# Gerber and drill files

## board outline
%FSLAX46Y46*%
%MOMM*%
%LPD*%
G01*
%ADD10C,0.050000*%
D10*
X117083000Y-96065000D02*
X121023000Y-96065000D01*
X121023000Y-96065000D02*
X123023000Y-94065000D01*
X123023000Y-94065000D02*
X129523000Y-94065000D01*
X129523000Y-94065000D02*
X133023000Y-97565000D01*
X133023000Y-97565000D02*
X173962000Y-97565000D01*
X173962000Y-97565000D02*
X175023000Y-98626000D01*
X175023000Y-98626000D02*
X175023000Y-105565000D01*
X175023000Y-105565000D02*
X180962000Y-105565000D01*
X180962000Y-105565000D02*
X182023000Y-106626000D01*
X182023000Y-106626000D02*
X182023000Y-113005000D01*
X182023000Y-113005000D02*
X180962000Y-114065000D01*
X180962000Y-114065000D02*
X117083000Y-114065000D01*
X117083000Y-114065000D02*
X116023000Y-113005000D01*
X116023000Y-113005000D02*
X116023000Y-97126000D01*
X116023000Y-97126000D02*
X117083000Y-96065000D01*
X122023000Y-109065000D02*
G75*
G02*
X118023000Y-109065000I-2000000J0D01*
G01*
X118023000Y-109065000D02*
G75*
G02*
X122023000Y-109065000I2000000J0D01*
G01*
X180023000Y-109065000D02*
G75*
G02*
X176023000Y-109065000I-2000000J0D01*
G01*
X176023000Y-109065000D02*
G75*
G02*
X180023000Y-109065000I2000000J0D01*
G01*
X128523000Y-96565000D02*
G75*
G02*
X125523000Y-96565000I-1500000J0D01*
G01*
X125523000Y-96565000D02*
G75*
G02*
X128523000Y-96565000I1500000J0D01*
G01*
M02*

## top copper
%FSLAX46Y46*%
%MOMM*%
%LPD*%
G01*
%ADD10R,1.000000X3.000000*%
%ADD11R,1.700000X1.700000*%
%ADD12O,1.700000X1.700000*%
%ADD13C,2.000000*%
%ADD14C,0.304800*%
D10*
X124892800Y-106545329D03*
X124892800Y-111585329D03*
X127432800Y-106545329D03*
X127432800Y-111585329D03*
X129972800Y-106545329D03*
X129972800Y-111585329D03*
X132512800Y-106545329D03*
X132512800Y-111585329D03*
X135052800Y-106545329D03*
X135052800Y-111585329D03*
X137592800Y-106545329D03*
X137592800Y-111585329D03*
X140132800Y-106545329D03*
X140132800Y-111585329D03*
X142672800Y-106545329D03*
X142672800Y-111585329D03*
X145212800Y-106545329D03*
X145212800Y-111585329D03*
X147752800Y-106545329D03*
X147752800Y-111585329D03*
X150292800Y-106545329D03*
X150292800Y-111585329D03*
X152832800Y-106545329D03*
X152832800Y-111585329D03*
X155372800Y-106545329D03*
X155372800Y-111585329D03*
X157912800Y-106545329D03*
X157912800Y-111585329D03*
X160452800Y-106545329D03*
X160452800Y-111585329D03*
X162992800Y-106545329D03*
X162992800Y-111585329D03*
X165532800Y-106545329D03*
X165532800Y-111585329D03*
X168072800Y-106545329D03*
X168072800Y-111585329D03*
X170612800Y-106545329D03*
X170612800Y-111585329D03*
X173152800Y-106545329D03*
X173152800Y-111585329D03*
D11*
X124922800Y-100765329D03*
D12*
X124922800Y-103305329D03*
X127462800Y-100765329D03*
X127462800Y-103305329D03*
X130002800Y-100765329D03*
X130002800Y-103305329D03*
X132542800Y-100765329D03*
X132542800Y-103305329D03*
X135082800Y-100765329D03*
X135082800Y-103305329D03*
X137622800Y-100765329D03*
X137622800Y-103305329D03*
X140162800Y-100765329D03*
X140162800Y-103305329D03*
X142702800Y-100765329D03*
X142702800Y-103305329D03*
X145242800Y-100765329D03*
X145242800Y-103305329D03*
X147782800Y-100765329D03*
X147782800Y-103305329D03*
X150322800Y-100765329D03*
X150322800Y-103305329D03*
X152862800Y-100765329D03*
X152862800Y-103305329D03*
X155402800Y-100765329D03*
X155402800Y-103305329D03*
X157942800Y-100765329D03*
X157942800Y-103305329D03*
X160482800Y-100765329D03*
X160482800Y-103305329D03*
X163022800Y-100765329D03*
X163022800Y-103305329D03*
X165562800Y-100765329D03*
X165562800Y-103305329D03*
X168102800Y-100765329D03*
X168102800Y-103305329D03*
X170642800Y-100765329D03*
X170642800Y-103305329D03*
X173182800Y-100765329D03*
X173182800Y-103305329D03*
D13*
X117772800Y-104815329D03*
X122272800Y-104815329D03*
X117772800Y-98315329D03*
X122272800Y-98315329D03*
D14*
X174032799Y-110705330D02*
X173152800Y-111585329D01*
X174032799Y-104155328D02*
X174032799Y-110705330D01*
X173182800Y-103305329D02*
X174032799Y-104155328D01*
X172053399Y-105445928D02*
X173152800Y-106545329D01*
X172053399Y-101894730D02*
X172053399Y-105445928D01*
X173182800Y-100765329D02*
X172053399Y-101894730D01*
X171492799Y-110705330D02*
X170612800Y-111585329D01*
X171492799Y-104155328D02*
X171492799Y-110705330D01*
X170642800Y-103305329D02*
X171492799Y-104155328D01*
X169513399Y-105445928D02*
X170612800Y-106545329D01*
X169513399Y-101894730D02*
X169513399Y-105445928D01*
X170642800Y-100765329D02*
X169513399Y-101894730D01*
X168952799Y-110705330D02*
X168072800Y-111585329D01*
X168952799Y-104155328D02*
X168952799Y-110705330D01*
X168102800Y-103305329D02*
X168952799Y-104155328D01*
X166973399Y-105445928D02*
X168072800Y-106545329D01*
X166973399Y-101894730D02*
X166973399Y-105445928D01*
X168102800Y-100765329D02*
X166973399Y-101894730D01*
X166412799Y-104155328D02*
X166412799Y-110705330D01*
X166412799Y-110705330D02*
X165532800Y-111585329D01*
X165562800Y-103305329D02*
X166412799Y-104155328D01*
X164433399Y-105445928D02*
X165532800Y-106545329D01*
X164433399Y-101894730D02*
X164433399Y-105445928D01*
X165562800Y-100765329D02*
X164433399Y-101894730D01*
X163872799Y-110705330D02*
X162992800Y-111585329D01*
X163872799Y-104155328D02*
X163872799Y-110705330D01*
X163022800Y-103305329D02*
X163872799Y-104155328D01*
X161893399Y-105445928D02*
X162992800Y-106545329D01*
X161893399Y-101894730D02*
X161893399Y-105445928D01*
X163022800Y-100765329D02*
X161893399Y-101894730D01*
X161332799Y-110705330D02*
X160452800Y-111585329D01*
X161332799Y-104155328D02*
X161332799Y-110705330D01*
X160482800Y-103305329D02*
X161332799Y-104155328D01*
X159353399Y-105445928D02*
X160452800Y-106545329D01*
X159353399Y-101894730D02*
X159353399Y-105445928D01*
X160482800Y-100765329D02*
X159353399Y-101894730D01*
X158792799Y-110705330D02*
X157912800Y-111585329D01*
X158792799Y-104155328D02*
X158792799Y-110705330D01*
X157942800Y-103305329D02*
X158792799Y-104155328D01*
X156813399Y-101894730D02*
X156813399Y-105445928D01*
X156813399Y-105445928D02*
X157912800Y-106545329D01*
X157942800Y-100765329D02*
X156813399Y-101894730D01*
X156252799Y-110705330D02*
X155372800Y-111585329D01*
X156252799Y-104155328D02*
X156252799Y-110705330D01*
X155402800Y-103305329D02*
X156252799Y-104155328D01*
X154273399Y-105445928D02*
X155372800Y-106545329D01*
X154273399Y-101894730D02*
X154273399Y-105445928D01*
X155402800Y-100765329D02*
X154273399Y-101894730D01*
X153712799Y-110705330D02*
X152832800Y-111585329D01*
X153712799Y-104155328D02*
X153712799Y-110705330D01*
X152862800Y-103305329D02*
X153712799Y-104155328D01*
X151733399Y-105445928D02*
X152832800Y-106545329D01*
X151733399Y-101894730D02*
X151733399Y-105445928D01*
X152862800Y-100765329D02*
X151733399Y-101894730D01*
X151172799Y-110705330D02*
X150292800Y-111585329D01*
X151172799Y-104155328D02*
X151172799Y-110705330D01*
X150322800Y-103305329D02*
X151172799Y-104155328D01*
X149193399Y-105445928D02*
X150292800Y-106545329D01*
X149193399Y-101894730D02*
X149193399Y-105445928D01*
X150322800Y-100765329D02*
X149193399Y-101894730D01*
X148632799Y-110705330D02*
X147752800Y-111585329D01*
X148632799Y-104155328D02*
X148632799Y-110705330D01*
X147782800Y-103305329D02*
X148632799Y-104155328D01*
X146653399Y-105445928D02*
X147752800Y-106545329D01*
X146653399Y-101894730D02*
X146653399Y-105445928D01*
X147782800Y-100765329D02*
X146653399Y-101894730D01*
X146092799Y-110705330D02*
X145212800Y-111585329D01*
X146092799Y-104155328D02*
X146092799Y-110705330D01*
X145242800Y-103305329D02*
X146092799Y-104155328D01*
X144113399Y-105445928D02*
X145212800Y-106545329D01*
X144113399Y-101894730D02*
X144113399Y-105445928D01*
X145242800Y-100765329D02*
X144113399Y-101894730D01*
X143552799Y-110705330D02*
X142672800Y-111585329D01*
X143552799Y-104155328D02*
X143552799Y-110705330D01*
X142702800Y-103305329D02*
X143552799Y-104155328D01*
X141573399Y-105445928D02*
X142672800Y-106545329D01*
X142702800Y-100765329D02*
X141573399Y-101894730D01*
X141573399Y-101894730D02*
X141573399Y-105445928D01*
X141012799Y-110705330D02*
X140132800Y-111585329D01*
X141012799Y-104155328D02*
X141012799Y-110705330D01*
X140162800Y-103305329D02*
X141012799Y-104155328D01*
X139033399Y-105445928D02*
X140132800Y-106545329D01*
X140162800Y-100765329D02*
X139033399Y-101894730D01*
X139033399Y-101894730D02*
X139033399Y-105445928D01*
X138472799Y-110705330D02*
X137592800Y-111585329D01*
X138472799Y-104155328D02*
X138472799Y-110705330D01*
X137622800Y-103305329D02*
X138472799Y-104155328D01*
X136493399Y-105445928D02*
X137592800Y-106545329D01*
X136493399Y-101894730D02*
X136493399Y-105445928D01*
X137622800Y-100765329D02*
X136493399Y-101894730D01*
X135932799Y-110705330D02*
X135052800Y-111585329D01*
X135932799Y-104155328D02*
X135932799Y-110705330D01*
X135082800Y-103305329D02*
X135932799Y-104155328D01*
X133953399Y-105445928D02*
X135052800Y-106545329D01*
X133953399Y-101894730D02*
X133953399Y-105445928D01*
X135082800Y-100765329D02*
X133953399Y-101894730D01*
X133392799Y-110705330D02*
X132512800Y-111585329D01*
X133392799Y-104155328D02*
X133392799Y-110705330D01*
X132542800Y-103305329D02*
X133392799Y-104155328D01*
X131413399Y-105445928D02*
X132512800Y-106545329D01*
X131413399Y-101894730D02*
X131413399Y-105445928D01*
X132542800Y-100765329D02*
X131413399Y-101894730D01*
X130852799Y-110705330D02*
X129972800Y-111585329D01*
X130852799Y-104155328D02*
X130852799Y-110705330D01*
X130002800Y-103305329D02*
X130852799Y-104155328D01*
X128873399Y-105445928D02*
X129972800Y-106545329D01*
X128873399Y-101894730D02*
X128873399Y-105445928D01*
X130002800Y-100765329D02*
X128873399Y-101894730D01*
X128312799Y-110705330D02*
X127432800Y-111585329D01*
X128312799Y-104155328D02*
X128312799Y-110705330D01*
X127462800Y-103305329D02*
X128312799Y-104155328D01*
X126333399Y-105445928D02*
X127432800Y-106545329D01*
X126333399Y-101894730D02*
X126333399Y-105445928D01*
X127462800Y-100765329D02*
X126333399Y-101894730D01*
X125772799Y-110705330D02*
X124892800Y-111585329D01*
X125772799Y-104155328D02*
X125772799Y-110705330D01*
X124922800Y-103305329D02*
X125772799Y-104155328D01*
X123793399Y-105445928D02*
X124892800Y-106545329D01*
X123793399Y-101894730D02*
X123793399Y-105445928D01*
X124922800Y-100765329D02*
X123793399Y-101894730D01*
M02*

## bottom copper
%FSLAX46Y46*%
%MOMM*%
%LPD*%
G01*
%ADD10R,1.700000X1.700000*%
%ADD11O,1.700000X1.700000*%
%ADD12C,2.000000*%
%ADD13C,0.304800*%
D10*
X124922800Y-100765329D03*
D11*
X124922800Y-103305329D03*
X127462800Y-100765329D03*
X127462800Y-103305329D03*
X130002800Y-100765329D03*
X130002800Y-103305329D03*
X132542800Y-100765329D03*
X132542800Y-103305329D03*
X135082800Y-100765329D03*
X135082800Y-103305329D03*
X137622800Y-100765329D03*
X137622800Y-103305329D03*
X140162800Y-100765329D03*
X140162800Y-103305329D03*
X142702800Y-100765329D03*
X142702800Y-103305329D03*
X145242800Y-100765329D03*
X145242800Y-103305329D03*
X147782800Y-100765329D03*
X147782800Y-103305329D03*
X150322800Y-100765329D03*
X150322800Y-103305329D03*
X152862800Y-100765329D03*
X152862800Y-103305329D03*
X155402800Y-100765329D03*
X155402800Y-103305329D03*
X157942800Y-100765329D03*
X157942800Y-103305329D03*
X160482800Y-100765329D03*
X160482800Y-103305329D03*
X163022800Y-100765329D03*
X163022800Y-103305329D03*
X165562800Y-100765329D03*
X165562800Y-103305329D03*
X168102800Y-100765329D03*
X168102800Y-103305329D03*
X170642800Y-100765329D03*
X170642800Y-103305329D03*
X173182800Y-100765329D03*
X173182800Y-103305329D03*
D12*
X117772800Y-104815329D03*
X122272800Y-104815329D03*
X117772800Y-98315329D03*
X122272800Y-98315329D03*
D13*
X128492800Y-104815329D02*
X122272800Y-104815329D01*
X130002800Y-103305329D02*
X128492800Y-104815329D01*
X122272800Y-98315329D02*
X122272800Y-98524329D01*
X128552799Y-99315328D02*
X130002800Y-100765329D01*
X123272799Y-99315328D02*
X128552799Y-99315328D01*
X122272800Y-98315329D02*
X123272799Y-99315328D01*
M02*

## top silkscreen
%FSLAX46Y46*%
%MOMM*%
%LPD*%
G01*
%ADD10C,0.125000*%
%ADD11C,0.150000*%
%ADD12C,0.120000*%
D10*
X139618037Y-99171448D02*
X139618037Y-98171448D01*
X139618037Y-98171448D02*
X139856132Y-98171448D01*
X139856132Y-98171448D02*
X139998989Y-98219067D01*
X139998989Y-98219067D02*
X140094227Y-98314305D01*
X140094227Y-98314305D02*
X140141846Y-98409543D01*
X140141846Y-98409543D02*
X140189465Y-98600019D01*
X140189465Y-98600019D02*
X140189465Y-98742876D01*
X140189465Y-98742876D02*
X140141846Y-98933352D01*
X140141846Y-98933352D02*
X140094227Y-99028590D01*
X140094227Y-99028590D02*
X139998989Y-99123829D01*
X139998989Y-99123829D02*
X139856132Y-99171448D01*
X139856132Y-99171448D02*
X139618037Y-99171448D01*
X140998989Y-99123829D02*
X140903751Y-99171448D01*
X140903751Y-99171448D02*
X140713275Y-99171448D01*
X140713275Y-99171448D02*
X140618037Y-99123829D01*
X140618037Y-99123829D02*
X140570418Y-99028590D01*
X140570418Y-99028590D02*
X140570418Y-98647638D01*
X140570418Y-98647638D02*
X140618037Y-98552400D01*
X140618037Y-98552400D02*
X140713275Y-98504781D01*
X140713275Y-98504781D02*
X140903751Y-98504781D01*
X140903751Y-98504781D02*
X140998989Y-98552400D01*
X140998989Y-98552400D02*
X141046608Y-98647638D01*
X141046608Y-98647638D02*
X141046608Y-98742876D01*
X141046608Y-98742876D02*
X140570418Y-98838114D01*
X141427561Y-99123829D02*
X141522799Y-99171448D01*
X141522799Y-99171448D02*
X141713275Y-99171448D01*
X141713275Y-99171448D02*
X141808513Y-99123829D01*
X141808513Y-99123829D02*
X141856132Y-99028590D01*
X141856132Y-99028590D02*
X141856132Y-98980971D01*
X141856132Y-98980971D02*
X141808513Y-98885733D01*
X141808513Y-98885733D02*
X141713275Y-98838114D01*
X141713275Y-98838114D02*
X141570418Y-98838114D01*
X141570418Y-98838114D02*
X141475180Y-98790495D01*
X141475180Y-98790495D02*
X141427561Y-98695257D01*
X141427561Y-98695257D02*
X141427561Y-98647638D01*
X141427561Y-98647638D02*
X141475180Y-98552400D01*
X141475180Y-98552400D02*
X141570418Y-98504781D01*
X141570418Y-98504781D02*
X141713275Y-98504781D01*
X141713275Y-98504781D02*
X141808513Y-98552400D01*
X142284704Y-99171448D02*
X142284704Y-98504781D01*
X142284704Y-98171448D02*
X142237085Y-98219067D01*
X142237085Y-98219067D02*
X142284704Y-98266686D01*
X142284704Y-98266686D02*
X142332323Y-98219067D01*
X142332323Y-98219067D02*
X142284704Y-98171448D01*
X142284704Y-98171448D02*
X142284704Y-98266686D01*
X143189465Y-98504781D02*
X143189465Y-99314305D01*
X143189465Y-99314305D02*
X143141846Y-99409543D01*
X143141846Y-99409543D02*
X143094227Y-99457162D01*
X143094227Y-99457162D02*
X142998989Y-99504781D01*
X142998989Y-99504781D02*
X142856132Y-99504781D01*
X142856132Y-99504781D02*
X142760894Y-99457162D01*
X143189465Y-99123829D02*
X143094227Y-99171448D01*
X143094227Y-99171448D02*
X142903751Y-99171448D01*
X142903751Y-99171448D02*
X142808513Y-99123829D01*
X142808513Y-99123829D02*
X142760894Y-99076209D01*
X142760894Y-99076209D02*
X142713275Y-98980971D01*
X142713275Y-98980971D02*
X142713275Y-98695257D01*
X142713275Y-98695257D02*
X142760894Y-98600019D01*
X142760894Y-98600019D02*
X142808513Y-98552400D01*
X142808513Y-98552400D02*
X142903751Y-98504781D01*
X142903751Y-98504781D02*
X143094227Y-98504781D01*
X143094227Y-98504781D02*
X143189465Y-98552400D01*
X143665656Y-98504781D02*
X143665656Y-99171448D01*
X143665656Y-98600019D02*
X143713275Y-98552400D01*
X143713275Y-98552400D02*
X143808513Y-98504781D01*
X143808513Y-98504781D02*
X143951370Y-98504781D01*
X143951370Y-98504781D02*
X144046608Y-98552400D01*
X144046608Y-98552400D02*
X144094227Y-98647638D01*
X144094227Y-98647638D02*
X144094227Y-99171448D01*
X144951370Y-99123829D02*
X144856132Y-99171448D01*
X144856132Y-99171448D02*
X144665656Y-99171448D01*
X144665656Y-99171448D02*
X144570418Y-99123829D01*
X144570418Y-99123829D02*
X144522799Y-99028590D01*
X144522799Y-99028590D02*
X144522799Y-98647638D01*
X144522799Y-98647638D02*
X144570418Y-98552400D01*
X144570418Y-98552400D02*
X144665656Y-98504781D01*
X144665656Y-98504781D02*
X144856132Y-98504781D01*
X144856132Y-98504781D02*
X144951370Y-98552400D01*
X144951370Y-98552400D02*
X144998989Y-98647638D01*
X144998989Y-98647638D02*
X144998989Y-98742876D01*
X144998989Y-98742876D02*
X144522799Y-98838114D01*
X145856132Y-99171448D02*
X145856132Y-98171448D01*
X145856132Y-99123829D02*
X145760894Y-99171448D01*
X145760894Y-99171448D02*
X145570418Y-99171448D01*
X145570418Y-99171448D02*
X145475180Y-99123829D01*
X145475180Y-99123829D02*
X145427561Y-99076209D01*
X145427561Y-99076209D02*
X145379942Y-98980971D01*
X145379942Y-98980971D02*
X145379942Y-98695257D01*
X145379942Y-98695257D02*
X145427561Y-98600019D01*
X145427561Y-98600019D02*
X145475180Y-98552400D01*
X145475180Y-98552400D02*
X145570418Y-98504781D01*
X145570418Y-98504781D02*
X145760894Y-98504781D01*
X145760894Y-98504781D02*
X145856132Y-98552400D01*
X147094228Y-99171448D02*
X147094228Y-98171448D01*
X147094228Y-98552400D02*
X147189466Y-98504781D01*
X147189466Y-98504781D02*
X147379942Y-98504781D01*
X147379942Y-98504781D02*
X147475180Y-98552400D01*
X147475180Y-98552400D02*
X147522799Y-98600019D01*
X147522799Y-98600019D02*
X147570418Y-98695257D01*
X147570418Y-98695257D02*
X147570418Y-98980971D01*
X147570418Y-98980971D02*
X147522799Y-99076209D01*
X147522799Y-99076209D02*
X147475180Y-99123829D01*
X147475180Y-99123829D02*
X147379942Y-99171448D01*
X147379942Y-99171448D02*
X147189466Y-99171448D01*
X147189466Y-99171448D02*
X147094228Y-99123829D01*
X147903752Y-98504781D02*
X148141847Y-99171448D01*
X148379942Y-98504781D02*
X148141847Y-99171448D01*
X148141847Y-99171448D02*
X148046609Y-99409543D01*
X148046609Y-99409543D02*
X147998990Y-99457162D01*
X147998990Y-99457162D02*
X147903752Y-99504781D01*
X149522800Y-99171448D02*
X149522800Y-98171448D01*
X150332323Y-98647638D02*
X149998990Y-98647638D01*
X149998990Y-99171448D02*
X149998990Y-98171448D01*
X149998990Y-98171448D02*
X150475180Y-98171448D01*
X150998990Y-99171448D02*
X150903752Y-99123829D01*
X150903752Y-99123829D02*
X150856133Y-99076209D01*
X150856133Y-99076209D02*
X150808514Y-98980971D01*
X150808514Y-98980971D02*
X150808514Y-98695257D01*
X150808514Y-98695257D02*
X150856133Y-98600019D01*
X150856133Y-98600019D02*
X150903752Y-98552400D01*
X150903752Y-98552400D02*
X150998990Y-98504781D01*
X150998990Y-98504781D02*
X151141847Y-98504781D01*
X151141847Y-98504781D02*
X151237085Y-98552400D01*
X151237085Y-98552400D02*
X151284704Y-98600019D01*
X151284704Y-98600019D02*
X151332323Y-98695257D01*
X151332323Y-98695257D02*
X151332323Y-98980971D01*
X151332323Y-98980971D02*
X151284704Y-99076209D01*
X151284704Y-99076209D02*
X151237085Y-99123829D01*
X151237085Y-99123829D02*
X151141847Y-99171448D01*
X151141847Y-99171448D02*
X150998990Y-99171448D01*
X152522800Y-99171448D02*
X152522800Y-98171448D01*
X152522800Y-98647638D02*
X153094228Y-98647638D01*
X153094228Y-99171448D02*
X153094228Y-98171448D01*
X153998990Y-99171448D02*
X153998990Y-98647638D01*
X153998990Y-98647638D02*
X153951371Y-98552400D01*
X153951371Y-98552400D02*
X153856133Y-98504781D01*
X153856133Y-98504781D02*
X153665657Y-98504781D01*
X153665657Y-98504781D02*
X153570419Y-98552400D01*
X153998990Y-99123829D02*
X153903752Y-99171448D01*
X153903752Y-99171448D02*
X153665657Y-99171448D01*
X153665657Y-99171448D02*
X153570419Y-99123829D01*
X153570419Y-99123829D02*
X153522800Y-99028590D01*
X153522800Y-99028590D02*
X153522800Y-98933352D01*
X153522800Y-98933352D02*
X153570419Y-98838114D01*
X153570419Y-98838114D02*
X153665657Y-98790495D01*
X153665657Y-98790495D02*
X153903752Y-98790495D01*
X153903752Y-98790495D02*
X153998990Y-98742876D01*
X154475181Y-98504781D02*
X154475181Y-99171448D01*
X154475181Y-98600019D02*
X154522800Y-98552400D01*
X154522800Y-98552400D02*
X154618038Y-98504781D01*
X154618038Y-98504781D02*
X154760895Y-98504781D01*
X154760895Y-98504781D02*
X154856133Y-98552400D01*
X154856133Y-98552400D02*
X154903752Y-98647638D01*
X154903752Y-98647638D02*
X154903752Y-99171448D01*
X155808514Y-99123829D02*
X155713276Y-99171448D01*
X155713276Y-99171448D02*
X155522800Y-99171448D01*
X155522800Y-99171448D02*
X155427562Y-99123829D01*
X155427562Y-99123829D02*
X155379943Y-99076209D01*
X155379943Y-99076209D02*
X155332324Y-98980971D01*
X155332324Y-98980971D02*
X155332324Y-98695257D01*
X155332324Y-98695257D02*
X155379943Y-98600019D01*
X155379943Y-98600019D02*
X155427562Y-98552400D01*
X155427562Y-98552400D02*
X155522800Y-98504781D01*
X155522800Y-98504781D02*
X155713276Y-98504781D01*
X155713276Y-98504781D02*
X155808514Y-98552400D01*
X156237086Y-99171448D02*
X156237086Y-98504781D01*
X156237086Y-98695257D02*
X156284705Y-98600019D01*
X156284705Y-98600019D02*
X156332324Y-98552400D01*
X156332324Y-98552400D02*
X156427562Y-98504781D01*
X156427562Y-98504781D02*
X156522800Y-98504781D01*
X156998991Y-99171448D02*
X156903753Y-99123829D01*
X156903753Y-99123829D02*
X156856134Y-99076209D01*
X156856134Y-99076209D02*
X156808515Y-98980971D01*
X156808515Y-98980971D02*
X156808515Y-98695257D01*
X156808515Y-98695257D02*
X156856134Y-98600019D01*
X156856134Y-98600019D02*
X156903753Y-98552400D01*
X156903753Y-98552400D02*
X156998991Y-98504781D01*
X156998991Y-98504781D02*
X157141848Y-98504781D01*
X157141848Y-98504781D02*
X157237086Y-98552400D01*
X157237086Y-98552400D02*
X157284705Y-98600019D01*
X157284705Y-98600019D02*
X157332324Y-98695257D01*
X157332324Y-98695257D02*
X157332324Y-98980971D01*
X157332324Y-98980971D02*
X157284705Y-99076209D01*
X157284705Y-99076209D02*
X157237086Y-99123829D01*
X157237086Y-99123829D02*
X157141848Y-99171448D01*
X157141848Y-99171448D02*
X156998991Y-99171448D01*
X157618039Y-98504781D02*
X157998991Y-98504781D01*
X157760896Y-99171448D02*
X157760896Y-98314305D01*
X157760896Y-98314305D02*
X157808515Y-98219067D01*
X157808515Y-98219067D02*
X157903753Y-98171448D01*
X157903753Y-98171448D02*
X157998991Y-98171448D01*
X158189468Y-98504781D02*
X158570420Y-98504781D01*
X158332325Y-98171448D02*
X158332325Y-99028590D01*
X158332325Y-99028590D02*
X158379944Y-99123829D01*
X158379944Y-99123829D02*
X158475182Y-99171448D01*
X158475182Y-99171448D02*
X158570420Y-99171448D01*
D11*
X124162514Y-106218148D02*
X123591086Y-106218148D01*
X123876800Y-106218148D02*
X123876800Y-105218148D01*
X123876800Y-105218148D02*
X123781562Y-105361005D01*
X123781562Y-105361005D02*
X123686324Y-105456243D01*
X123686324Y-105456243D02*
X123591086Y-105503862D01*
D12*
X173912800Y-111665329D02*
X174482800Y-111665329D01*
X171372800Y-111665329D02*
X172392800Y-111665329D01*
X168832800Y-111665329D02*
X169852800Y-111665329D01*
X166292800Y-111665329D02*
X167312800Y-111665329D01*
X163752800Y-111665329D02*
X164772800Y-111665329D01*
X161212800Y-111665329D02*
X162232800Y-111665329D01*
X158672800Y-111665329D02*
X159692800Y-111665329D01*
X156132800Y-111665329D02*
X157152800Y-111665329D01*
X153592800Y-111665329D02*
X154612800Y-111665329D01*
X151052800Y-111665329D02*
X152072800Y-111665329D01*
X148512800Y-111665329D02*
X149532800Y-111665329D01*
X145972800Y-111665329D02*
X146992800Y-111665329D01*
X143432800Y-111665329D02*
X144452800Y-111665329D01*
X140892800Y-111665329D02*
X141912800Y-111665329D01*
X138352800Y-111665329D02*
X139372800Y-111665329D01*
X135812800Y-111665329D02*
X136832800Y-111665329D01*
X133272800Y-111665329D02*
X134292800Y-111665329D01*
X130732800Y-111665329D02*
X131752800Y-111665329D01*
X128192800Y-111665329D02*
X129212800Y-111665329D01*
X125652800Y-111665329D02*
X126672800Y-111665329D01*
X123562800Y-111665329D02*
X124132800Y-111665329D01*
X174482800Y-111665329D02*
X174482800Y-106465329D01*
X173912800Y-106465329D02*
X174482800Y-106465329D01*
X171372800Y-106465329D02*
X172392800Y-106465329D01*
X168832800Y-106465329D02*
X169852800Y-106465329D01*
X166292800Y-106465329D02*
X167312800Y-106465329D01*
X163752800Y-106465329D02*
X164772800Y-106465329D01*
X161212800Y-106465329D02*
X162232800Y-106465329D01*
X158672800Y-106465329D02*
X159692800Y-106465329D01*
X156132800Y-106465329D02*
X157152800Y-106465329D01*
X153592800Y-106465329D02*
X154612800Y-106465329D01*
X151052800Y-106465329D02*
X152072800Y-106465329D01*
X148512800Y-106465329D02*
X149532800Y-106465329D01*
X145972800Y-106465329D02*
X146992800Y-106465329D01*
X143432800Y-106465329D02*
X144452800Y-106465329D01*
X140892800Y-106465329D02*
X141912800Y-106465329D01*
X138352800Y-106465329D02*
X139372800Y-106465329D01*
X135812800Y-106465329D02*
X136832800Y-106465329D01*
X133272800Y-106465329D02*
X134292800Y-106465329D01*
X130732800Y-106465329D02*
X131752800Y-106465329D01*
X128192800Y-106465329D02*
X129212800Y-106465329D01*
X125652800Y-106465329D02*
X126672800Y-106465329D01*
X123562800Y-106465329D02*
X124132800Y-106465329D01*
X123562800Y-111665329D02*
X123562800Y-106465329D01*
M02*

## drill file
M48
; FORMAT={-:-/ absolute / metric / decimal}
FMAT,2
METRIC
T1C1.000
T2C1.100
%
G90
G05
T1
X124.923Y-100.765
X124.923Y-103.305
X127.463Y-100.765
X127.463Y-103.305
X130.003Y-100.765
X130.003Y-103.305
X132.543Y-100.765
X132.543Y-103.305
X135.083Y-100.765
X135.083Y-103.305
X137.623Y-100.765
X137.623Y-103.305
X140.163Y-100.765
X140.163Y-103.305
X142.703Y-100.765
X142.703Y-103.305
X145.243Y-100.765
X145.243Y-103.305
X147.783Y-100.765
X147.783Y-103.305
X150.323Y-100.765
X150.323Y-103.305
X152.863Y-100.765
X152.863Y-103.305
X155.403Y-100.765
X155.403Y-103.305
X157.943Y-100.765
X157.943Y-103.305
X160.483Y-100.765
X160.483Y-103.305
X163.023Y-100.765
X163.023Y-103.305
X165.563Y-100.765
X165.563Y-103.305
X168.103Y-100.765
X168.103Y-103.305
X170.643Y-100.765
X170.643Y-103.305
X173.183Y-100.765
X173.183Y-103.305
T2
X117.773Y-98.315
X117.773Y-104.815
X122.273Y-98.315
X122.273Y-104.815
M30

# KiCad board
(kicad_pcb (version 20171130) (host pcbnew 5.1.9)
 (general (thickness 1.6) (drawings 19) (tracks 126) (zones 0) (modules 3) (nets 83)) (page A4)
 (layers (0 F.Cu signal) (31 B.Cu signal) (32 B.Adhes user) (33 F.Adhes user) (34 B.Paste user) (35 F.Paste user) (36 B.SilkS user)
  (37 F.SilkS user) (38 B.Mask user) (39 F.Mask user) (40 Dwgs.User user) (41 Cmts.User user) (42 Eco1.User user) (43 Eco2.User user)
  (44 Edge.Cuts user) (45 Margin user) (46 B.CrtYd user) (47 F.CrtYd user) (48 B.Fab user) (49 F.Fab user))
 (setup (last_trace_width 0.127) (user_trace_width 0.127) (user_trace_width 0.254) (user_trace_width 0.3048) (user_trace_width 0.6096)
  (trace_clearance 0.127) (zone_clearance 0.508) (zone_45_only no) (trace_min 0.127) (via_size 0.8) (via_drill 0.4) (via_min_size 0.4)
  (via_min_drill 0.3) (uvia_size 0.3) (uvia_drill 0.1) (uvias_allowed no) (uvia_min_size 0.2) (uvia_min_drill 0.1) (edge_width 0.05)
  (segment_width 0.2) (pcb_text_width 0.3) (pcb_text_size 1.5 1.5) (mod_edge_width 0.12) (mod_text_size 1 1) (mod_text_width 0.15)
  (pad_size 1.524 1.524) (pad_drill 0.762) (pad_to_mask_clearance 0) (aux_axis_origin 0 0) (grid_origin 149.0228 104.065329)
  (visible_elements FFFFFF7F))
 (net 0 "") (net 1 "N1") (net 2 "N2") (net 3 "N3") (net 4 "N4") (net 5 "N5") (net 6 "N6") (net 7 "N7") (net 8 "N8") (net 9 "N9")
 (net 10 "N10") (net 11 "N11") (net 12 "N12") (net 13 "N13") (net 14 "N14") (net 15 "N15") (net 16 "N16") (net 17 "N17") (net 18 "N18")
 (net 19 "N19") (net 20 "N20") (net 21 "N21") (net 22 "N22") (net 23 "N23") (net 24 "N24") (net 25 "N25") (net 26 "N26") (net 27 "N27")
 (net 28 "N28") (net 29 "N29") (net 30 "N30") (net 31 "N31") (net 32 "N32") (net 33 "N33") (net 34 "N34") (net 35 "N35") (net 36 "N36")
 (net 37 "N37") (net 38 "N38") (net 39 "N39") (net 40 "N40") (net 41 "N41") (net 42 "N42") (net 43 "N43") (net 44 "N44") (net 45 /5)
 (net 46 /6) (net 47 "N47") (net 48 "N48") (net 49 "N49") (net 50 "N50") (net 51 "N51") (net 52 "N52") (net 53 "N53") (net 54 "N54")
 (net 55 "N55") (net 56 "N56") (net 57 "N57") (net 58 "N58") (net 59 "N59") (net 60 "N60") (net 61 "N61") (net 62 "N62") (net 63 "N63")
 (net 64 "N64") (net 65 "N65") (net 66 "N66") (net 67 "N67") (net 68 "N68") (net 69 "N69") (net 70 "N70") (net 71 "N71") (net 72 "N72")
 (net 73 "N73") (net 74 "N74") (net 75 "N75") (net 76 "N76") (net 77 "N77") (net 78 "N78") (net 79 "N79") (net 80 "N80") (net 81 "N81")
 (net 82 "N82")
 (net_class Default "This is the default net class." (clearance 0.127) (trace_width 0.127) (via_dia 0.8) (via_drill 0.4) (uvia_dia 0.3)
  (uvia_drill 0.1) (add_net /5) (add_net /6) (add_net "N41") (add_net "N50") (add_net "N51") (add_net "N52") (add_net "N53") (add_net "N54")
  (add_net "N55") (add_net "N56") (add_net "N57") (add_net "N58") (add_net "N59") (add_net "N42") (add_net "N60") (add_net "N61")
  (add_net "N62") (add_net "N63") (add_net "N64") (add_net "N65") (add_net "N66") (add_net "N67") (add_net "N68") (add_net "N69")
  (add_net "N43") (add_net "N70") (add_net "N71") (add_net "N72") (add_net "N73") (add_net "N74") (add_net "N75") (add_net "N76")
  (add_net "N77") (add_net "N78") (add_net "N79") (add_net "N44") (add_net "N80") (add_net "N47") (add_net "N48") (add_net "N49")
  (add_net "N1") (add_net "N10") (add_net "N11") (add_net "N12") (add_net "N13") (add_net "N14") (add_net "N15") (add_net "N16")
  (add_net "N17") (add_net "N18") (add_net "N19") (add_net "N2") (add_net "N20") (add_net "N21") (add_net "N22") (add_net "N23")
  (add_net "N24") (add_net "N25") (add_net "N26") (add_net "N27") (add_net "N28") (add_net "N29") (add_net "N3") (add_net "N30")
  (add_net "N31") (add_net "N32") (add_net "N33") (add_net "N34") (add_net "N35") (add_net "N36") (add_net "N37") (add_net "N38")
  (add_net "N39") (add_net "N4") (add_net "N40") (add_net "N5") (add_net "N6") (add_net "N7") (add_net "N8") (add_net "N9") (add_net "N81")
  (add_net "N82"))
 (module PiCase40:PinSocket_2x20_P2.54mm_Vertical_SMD (layer F.Cu) (at 149.0228 109.065329 90)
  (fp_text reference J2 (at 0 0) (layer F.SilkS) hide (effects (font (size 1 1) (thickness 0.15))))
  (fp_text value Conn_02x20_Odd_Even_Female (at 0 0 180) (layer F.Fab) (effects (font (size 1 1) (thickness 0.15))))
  (fp_line (start -2.6 24.89) (end -2.6 25.46) (layer F.SilkS) (width 0.12))
  (fp_line (start -2.6 22.35) (end -2.6 23.37) (layer F.SilkS) (width 0.12))
  (fp_line (start -2.6 19.81) (end -2.6 20.83) (layer F.SilkS) (width 0.12))
  (fp_line (start -2.6 17.27) (end -2.6 18.29) (layer F.SilkS) (width 0.12))
  (fp_line (start -2.6 14.73) (end -2.6 15.75) (layer F.SilkS) (width 0.12))
  (fp_line (start -2.6 12.19) (end -2.6 13.21) (layer F.SilkS) (width 0.12))
  (fp_line (start -2.6 9.65) (end -2.6 10.67) (layer F.SilkS) (width 0.12))
  (fp_line (start -2.6 7.11) (end -2.6 8.13) (layer F.SilkS) (width 0.12))
  (fp_line (start -2.6 4.57) (end -2.6 5.59) (layer F.SilkS) (width 0.12))
  (fp_line (start -2.6 2.03) (end -2.6 3.05) (layer F.SilkS) (width 0.12))
  (fp_line (start -2.6 -0.51) (end -2.6 0.51) (layer F.SilkS) (width 0.12))
  (fp_line (start -2.6 -3.05) (end -2.6 -2.03) (layer F.SilkS) (width 0.12))
  (fp_line (start -2.6 -5.59) (end -2.6 -4.57) (layer F.SilkS) (width 0.12))
  (fp_line (start -2.6 -8.13) (end -2.6 -7.11) (layer F.SilkS) (width 0.12))
  (fp_line (start -2.6 -10.67) (end -2.6 -9.65) (layer F.SilkS) (width 0.12))
  (fp_line (start -2.6 -13.21) (end -2.6 -12.19) (layer F.SilkS) (width 0.12))
  (fp_line (start -2.6 -15.75) (end -2.6 -14.73) (layer F.SilkS) (width 0.12))
  (fp_line (start -2.6 -18.29) (end -2.6 -17.27) (layer F.SilkS) (width 0.12))
  (fp_line (start -2.6 -20.83) (end -2.6 -19.81) (layer F.SilkS) (width 0.12))
  (fp_line (start -2.6 -23.37) (end -2.6 -22.35) (layer F.SilkS) (width 0.12))
  (fp_line (start -2.6 -25.46) (end -2.6 -24.89) (layer F.SilkS) (width 0.12))
  (fp_line (start -2.6 25.46) (end 2.6 25.46) (layer F.SilkS) (width 0.12))
  (fp_line (start 2.6 24.89) (end 2.6 25.46) (layer F.SilkS) (width 0.12))
  (fp_line (start 2.6 22.35) (end 2.6 23.37) (layer F.SilkS) (width 0.12))
  (fp_line (start 2.6 19.81) (end 2.6 20.83) (layer F.SilkS) (width 0.12))
  (fp_line (start 2.6 17.27) (end 2.6 18.29) (layer F.SilkS) (width 0.12))
  (fp_line (start 2.6 14.73) (end 2.6 15.75) (layer F.SilkS) (width 0.12))
  (fp_line (start 2.6 12.19) (end 2.6 13.21) (layer F.SilkS) (width 0.12))
  (fp_line (start 2.6 9.65) (end 2.6 10.67) (layer F.SilkS) (width 0.12))
  (fp_line (start 2.6 7.11) (end 2.6 8.13) (layer F.SilkS) (width 0.12))
  (fp_line (start 2.6 4.57) (end 2.6 5.59) (layer F.SilkS) (width 0.12))
  (fp_line (start 2.6 2.03) (end 2.6 3.05) (layer F.SilkS) (width 0.12))
  (fp_line (start 2.6 -0.51) (end 2.6 0.51) (layer F.SilkS) (width 0.12))
  (fp_line (start 2.6 -3.05) (end 2.6 -2.03) (layer F.SilkS) (width 0.12))
  (fp_line (start 2.6 -5.59) (end 2.6 -4.57) (layer F.SilkS) (width 0.12))
  (fp_line (start 2.6 -8.13) (end 2.6 -7.11) (layer F.SilkS) (width 0.12))
  (fp_line (start 2.6 -10.67) (end 2.6 -9.65) (layer F.SilkS) (width 0.12))
  (fp_line (start 2.6 -13.21) (end 2.6 -12.19) (layer F.SilkS) (width 0.12))
  (fp_line (start 2.6 -15.75) (end 2.6 -14.73) (layer F.SilkS) (width 0.12))
  (fp_line (start 2.6 -18.29) (end 2.6 -17.27) (layer F.SilkS) (width 0.12))
  (fp_line (start 2.6 -20.83) (end 2.6 -19.81) (layer F.SilkS) (width 0.12))
  (fp_line (start 2.6 -23.37) (end 2.6 -22.35) (layer F.SilkS) (width 0.12))
  (fp_line (start 2.6 -25.46) (end 2.6 -24.89) (layer F.SilkS) (width 0.12))
  (fp_line (start -2.6 -25.46) (end 2.6 -25.46) (layer F.SilkS) (width 0.12))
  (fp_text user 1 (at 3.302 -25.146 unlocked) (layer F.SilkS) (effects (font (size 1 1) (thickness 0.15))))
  (pad 1 smd rect (at 2.52 -24.13 90) (size 3 1) (layers F.Cu F.Paste F.Mask) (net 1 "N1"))
  (pad 2 smd rect (at -2.52 -24.13 90) (size 3 1) (layers F.Cu F.Paste F.Mask) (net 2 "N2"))
  (pad 3 smd rect (at 2.52 -21.59 90) (size 3 1) (layers F.Cu F.Paste F.Mask) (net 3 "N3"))
  (pad 4 smd rect (at -2.52 -21.59 90) (size 3 1) (layers F.Cu F.Paste F.Mask) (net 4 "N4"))
  (pad 5 smd rect (at 2.52 -19.05 90) (size 3 1) (layers F.Cu F.Paste F.Mask) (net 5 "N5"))
  (pad 6 smd rect (at -2.52 -19.05 90) (size 3 1) (layers F.Cu F.Paste F.Mask) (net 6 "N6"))
  (pad 7 smd rect (at 2.52 -16.51 90) (size 3 1) (layers F.Cu F.Paste F.Mask) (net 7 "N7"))
  (pad 8 smd rect (at -2.52 -16.51 90) (size 3 1) (layers F.Cu F.Paste F.Mask) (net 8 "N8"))
  (pad 9 smd rect (at 2.52 -13.97 90) (size 3 1) (layers F.Cu F.Paste F.Mask) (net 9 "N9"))
  (pad 10 smd rect (at -2.52 -13.97 90) (size 3 1) (layers F.Cu F.Paste F.Mask) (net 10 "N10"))
  (pad 11 smd rect (at 2.52 -11.43 90) (size 3 1) (layers F.Cu F.Paste F.Mask) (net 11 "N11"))
  (pad 12 smd rect (at -2.52 -11.43 90) (size 3 1) (layers F.Cu F.Paste F.Mask) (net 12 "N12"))
  (pad 13 smd rect (at 2.52 -8.89 90) (size 3 1) (layers F.Cu F.Paste F.Mask) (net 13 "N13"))
  (pad 14 smd rect (at -2.52 -8.89 90) (size 3 1) (layers F.Cu F.Paste F.Mask) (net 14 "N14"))
  (pad 15 smd rect (at 2.52 -6.35 90) (size 3 1) (layers F.Cu F.Paste F.Mask) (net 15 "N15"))
  (pad 16 smd rect (at -2.52 -6.35 90) (size 3 1) (layers F.Cu F.Paste F.Mask) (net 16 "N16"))
  (pad 17 smd rect (at 2.52 -3.81 90) (size 3 1) (layers F.Cu F.Paste F.Mask) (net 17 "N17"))
  (pad 18 smd rect (at -2.52 -3.81 90) (size 3 1) (layers F.Cu F.Paste F.Mask) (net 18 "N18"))
  (pad 19 smd rect (at 2.52 -1.27 90) (size 3 1) (layers F.Cu F.Paste F.Mask) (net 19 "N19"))
  (pad 20 smd rect (at -2.52 -1.27 90) (size 3 1) (layers F.Cu F.Paste F.Mask) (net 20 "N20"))
  (pad 21 smd rect (at 2.52 1.27 90) (size 3 1) (layers F.Cu F.Paste F.Mask) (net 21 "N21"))
  (pad 22 smd rect (at -2.52 1.27 90) (size 3 1) (layers F.Cu F.Paste F.Mask) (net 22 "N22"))
  (pad 23 smd rect (at 2.52 3.81 90) (size 3 1) (layers F.Cu F.Paste F.Mask) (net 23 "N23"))
  (pad 24 smd rect (at -2.52 3.81 90) (size 3 1) (layers F.Cu F.Paste F.Mask) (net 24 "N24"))
  (pad 25 smd rect (at 2.52 6.35 90) (size 3 1) (layers F.Cu F.Paste F.Mask) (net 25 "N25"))
  (pad 26 smd rect (at -2.52 6.35 90) (size 3 1) (layers F.Cu F.Paste F.Mask) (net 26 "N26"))
  (pad 27 smd rect (at 2.52 8.89 90) (size 3 1) (layers F.Cu F.Paste F.Mask) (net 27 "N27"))
  (pad 28 smd rect (at -2.52 8.89 90) (size 3 1) (layers F.Cu F.Paste F.Mask) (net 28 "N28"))
  (pad 29 smd rect (at 2.52 11.43 90) (size 3 1) (layers F.Cu F.Paste F.Mask) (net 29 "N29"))
  (pad 30 smd rect (at -2.52 11.43 90) (size 3 1) (layers F.Cu F.Paste F.Mask) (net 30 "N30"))
  (pad 31 smd rect (at 2.52 13.97 90) (size 3 1) (layers F.Cu F.Paste F.Mask) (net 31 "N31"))
  (pad 32 smd rect (at -2.52 13.97 90) (size 3 1) (layers F.Cu F.Paste F.Mask) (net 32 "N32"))
  (pad 33 smd rect (at 2.52 16.51 90) (size 3 1) (layers F.Cu F.Paste F.Mask) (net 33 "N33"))
  (pad 34 smd rect (at -2.52 16.51 90) (size 3 1) (layers F.Cu F.Paste F.Mask) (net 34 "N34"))
  (pad 35 smd rect (at 2.52 19.05 90) (size 3 1) (layers F.Cu F.Paste F.Mask) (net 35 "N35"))
  (pad 36 smd rect (at -2.52 19.05 90) (size 3 1) (layers F.Cu F.Paste F.Mask) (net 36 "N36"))
  (pad 37 smd rect (at 2.52 21.59 90) (size 3 1) (layers F.Cu F.Paste F.Mask) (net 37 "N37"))
  (pad 38 smd rect (at -2.52 21.59 90) (size 3 1) (layers F.Cu F.Paste F.Mask) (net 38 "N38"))
  (pad 39 smd rect (at 2.52 24.13 90) (size 3 1) (layers F.Cu F.Paste F.Mask) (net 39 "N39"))
  (pad 40 smd rect (at -2.52 24.13 90) (size 3 1) (layers F.Cu F.Paste F.Mask) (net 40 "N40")))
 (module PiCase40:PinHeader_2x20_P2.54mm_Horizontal (layer B.Cu) (at 149.0228 102.065329 270)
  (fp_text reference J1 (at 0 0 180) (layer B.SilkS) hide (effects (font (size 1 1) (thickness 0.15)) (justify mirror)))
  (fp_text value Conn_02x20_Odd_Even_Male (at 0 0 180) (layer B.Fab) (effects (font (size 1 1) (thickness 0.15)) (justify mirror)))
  (pad 1 thru_hole rect (at -1.3 24.1 270) (size 1.7 1.7) (drill 1) (layers *.Cu *.Mask) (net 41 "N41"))
  (pad 2 thru_hole oval (at 1.24 24.1 270) (size 1.7 1.7) (drill 1) (layers *.Cu *.Mask) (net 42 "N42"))
  (pad 3 thru_hole oval (at -1.3 21.56 270) (size 1.7 1.7) (drill 1) (layers *.Cu *.Mask) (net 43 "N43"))
  (pad 4 thru_hole oval (at 1.24 21.56 270) (size 1.7 1.7) (drill 1) (layers *.Cu *.Mask) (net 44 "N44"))
  (pad 5 thru_hole oval (at -1.3 19.02 270) (size 1.7 1.7) (drill 1) (layers *.Cu *.Mask) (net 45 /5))
  (pad 6 thru_hole oval (at 1.24 19.02 270) (size 1.7 1.7) (drill 1) (layers *.Cu *.Mask) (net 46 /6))
  (pad 7 thru_hole oval (at -1.3 16.48 270) (size 1.7 1.7) (drill 1) (layers *.Cu *.Mask) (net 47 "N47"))
  (pad 8 thru_hole oval (at 1.24 16.48 270) (size 1.7 1.7) (drill 1) (layers *.Cu *.Mask) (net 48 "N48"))
  (pad 9 thru_hole oval (at -1.3 13.94 270) (size 1.7 1.7) (drill 1) (layers *.Cu *.Mask) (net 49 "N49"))
  (pad 10 thru_hole oval (at 1.24 13.94 270) (size 1.7 1.7) (drill 1) (layers *.Cu *.Mask) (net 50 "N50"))
  (pad 11 thru_hole oval (at -1.3 11.4 270) (size 1.7 1.7) (drill 1) (layers *.Cu *.Mask) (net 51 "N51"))
  (pad 12 thru_hole oval (at 1.24 11.4 270) (size 1.7 1.7) (drill 1) (layers *.Cu *.Mask) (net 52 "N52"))
  (pad 13 thru_hole oval (at -1.3 8.86 270) (size 1.7 1.7) (drill 1) (layers *.Cu *.Mask) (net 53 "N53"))
  (pad 14 thru_hole oval (at 1.24 8.86 270) (size 1.7 1.7) (drill 1) (layers *.Cu *.Mask) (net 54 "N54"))
  (pad 15 thru_hole oval (at -1.3 6.32 270) (size 1.7 1.7) (drill 1) (layers *.Cu *.Mask) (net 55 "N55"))
  (pad 16 thru_hole oval (at 1.24 6.32 270) (size 1.7 1.7) (drill 1) (layers *.Cu *.Mask) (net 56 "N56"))
  (pad 17 thru_hole oval (at -1.3 3.78 270) (size 1.7 1.7) (drill 1) (layers *.Cu *.Mask) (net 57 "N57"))
  (pad 18 thru_hole oval (at 1.24 3.78 270) (size 1.7 1.7) (drill 1) (layers *.Cu *.Mask) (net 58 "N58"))
  (pad 19 thru_hole oval (at -1.3 1.24 270) (size 1.7 1.7) (drill 1) (layers *.Cu *.Mask) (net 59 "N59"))
  (pad 20 thru_hole oval (at 1.24 1.24 270) (size 1.7 1.7) (drill 1) (layers *.Cu *.Mask) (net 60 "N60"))
  (pad 21 thru_hole oval (at -1.3 -1.3 270) (size 1.7 1.7) (drill 1) (layers *.Cu *.Mask) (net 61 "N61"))
  (pad 22 thru_hole oval (at 1.24 -1.3 270) (size 1.7 1.7) (drill 1) (layers *.Cu *.Mask) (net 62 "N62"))
  (pad 23 thru_hole oval (at -1.3 -3.84 270) (size 1.7 1.7) (drill 1) (layers *.Cu *.Mask) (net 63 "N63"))
  (pad 24 thru_hole oval (at 1.24 -3.84 270) (size 1.7 1.7) (drill 1) (layers *.Cu *.Mask) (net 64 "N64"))
  (pad 25 thru_hole oval (at -1.3 -6.38 270) (size 1.7 1.7) (drill 1) (layers *.Cu *.Mask) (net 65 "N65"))
  (pad 26 thru_hole oval (at 1.24 -6.38 270) (size 1.7 1.7) (drill 1) (layers *.Cu *.Mask) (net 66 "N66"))
  (pad 27 thru_hole oval (at -1.3 -8.92 270) (size 1.7 1.7) (drill 1) (layers *.Cu *.Mask) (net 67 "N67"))
  (pad 28 thru_hole oval (at 1.24 -8.92 270) (size 1.7 1.7) (drill 1) (layers *.Cu *.Mask) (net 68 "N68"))
  (pad 29 thru_hole oval (at -1.3 -11.46 270) (size 1.7 1.7) (drill 1) (layers *.Cu *.Mask) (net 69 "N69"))
  (pad 30 thru_hole oval (at 1.24 -11.46 270) (size 1.7 1.7) (drill 1) (layers *.Cu *.Mask) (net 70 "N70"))
  (pad 31 thru_hole oval (at -1.3 -14 270) (size 1.7 1.7) (drill 1) (layers *.Cu *.Mask) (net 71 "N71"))
  (pad 32 thru_hole oval (at 1.24 -14 270) (size 1.7 1.7) (drill 1) (layers *.Cu *.Mask) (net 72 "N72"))
  (pad 33 thru_hole oval (at -1.3 -16.54 270) (size 1.7 1.7) (drill 1) (layers *.Cu *.Mask) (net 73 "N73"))
  (pad 34 thru_hole oval (at 1.24 -16.54 270) (size 1.7 1.7) (drill 1) (layers *.Cu *.Mask) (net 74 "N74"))
  (pad 35 thru_hole oval (at -1.3 -19.08 270) (size 1.7 1.7) (drill 1) (layers *.Cu *.Mask) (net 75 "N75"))
  (pad 36 thru_hole oval (at 1.24 -19.08 270) (size 1.7 1.7) (drill 1) (layers *.Cu *.Mask) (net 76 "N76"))
  (pad 37 thru_hole oval (at -1.3 -21.62 270) (size 1.7 1.7) (drill 1) (layers *.Cu *.Mask) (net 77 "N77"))
  (pad 38 thru_hole oval (at 1.24 -21.62 270) (size 1.7 1.7) (drill 1) (layers *.Cu *.Mask) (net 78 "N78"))
  (pad 39 thru_hole oval (at -1.3 -24.16 270) (size 1.7 1.7) (drill 1) (layers *.Cu *.Mask) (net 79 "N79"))
  (pad 40 thru_hole oval (at 1.24 -24.16 270) (size 1.7 1.7) (drill 1) (layers *.Cu *.Mask) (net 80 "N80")))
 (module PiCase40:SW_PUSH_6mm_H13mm (layer B.Cu) (at 120.0228 101.565329 90)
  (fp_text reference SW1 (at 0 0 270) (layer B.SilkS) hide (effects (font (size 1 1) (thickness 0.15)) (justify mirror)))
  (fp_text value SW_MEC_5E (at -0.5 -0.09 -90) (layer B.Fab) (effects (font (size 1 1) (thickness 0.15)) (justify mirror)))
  (pad 2 thru_hole circle (at -3.25 -2.25) (size 2 2) (drill 1.1) (layers *.Cu *.Mask) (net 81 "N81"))
  (pad 3 thru_hole circle (at -3.25 2.25) (size 2 2) (drill 1.1) (layers *.Cu *.Mask) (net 46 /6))
  (pad 4 thru_hole circle (at 3.25 -2.25) (size 2 2) (drill 1.1) (layers *.Cu *.Mask) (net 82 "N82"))
  (pad 1 thru_hole circle (at 3.25 2.25) (size 2 2) (drill 1.1) (layers *.Cu *.Mask) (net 45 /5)))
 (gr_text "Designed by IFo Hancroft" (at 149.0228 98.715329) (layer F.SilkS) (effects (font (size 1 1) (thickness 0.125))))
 (gr_line (start 117.083 96.065) (end 121.023 96.065) (angle 90) (layer Edge.Cuts) (width 0.05))
 (gr_line (start 121.023 96.065) (end 123.023 94.065) (angle 90) (layer Edge.Cuts) (width 0.05))
 (gr_line (start 123.023 94.065) (end 129.523 94.065) (angle 90) (layer Edge.Cuts) (width 0.05))
 (gr_line (start 129.523 94.065) (end 133.023 97.565) (angle 90) (layer Edge.Cuts) (width 0.05))
 (gr_line (start 133.023 97.565) (end 173.962 97.565) (angle 90) (layer Edge.Cuts) (width 0.05))
 (gr_line (start 173.962 97.565) (end 175.023 98.626) (angle 90) (layer Edge.Cuts) (width 0.05))
 (gr_line (start 175.023 98.626) (end 175.023 105.565) (angle 90) (layer Edge.Cuts) (width 0.05))
 (gr_line (start 175.023 105.565) (end 180.962 105.565) (angle 90) (layer Edge.Cuts) (width 0.05))
 (gr_line (start 180.962 105.565) (end 182.023 106.626) (angle 90) (layer Edge.Cuts) (width 0.05))
 (gr_line (start 182.023 106.626) (end 182.023 113.005) (angle 90) (layer Edge.Cuts) (width 0.05))
 (gr_line (start 182.023 113.005) (end 180.962 114.065) (angle 90) (layer Edge.Cuts) (width 0.05))
 (gr_line (start 180.962 114.065) (end 117.083 114.065) (angle 90) (layer Edge.Cuts) (width 0.05))
 (gr_line (start 117.083 114.065) (end 116.023 113.005) (angle 90) (layer Edge.Cuts) (width 0.05))
 (gr_line (start 116.023 113.005) (end 116.023 97.126) (angle 90) (layer Edge.Cuts) (width 0.05))
 (gr_line (start 116.023 97.126) (end 117.083 96.065) (angle 90) (layer Edge.Cuts) (width 0.05))
 (gr_circle (center 120.023 109.065) (end 118.023 109.065) (layer Edge.Cuts) (width 0.05))
 (gr_circle (center 178.023 109.065) (end 176.023 109.065) (layer Edge.Cuts) (width 0.05))
 (gr_circle (center 127.023 96.565) (end 125.523 96.565) (layer Edge.Cuts) (width 0.05))
 (segment (start 174.032799 110.70533) (end 173.1528 111.585329) (width 0.3048) (layer F.Cu) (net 80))
 (segment (start 174.032799 104.155328) (end 174.032799 110.70533) (width 0.3048) (layer F.Cu) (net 80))
 (segment (start 173.1828 103.305329) (end 174.032799 104.155328) (width 0.3048) (layer F.Cu) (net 80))
 (segment (start 172.053399 105.445928) (end 173.1528 106.545329) (width 0.3048) (layer F.Cu) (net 79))
 (segment (start 172.053399 101.89473) (end 172.053399 105.445928) (width 0.3048) (layer F.Cu) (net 79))
 (segment (start 173.1828 100.765329) (end 172.053399 101.89473) (width 0.3048) (layer F.Cu) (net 79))
 (segment (start 171.492799 110.70533) (end 170.6128 111.585329) (width 0.3048) (layer F.Cu) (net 78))
 (segment (start 171.492799 104.155328) (end 171.492799 110.70533) (width 0.3048) (layer F.Cu) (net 78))
 (segment (start 170.6428 103.305329) (end 171.492799 104.155328) (width 0.3048) (layer F.Cu) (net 78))
 (segment (start 169.513399 105.445928) (end 170.6128 106.545329) (width 0.3048) (layer F.Cu) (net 77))
 (segment (start 169.513399 101.89473) (end 169.513399 105.445928) (width 0.3048) (layer F.Cu) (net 77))
 (segment (start 170.6428 100.765329) (end 169.513399 101.89473) (width 0.3048) (layer F.Cu) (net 77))
 (segment (start 168.952799 110.70533) (end 168.0728 111.585329) (width 0.3048) (layer F.Cu) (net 76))
 (segment (start 168.952799 104.155328) (end 168.952799 110.70533) (width 0.3048) (layer F.Cu) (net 76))
 (segment (start 168.1028 103.305329) (end 168.952799 104.155328) (width 0.3048) (layer F.Cu) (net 76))
 (segment (start 166.973399 105.445928) (end 168.0728 106.545329) (width 0.3048) (layer F.Cu) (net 75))
 (segment (start 166.973399 101.89473) (end 166.973399 105.445928) (width 0.3048) (layer F.Cu) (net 75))
 (segment (start 168.1028 100.765329) (end 166.973399 101.89473) (width 0.3048) (layer F.Cu) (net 75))
 (segment (start 166.412799 104.155328) (end 166.412799 110.70533) (width 0.3048) (layer F.Cu) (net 74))
 (segment (start 166.412799 110.70533) (end 165.5328 111.585329) (width 0.3048) (layer F.Cu) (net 74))
 (segment (start 165.5628 103.305329) (end 166.412799 104.155328) (width 0.3048) (layer F.Cu) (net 74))
 (segment (start 164.433399 105.445928) (end 165.5328 106.545329) (width 0.3048) (layer F.Cu) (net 73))
 (segment (start 164.433399 101.89473) (end 164.433399 105.445928) (width 0.3048) (layer F.Cu) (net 73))
 (segment (start 165.5628 100.765329) (end 164.433399 101.89473) (width 0.3048) (layer F.Cu) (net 73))
 (segment (start 163.872799 110.70533) (end 162.9928 111.585329) (width 0.3048) (layer F.Cu) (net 72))
 (segment (start 163.872799 104.155328) (end 163.872799 110.70533) (width 0.3048) (layer F.Cu) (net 72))
 (segment (start 163.0228 103.305329) (end 163.872799 104.155328) (width 0.3048) (layer F.Cu) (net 72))
 (segment (start 161.893399 105.445928) (end 162.9928 106.545329) (width 0.3048) (layer F.Cu) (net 71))
 (segment (start 161.893399 101.89473) (end 161.893399 105.445928) (width 0.3048) (layer F.Cu) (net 71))
 (segment (start 163.0228 100.765329) (end 161.893399 101.89473) (width 0.3048) (layer F.Cu) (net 71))
 (segment (start 161.332799 110.70533) (end 160.4528 111.585329) (width 0.3048) (layer F.Cu) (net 70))
 (segment (start 161.332799 104.155328) (end 161.332799 110.70533) (width 0.3048) (layer F.Cu) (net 70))
 (segment (start 160.4828 103.305329) (end 161.332799 104.155328) (width 0.3048) (layer F.Cu) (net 70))
 (segment (start 159.353399 105.445928) (end 160.4528 106.545329) (width 0.3048) (layer F.Cu) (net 69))
 (segment (start 159.353399 101.89473) (end 159.353399 105.445928) (width 0.3048) (layer F.Cu) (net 69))
 (segment (start 160.4828 100.765329) (end 159.353399 101.89473) (width 0.3048) (layer F.Cu) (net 69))
 (segment (start 158.792799 110.70533) (end 157.9128 111.585329) (width 0.3048) (layer F.Cu) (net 68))
 (segment (start 158.792799 104.155328) (end 158.792799 110.70533) (width 0.3048) (layer F.Cu) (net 68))
 (segment (start 157.9428 103.305329) (end 158.792799 104.155328) (width 0.3048) (layer F.Cu) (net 68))
 (segment (start 156.813399 101.89473) (end 156.813399 105.445928) (width 0.3048) (layer F.Cu) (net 67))
 (segment (start 156.813399 105.445928) (end 157.9128 106.545329) (width 0.3048) (layer F.Cu) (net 67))
 (segment (start 157.9428 100.765329) (end 156.813399 101.89473) (width 0.3048) (layer F.Cu) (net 67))
 (segment (start 156.252799 110.70533) (end 155.3728 111.585329) (width 0.3048) (layer F.Cu) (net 66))
 (segment (start 156.252799 104.155328) (end 156.252799 110.70533) (width 0.3048) (layer F.Cu) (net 66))
 (segment (start 155.4028 103.305329) (end 156.252799 104.155328) (width 0.3048) (layer F.Cu) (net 66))
 (segment (start 154.273399 105.445928) (end 155.3728 106.545329) (width 0.3048) (layer F.Cu) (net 65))
 (segment (start 154.273399 101.89473) (end 154.273399 105.445928) (width 0.3048) (layer F.Cu) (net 65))
 (segment (start 155.4028 100.765329) (end 154.273399 101.89473) (width 0.3048) (layer F.Cu) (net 65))
 (segment (start 153.712799 110.70533) (end 152.8328 111.585329) (width 0.3048) (layer F.Cu) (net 64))
 (segment (start 153.712799 104.155328) (end 153.712799 110.70533) (width 0.3048) (layer F.Cu) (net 64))
 (segment (start 152.8628 103.305329) (end 153.712799 104.155328) (width 0.3048) (layer F.Cu) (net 64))
 (segment (start 151.733399 105.445928) (end 152.8328 106.545329) (width 0.3048) (layer F.Cu) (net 63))
 (segment (start 151.733399 101.89473) (end 151.733399 105.445928) (width 0.3048) (layer F.Cu) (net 63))
 (segment (start 152.8628 100.765329) (end 151.733399 101.89473) (width 0.3048) (layer F.Cu) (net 63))
 (segment (start 151.172799 110.70533) (end 150.2928 111.585329) (width 0.3048) (layer F.Cu) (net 62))
 (segment (start 151.172799 104.155328) (end 151.172799 110.70533) (width 0.3048) (layer F.Cu) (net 62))
 (segment (start 150.3228 103.305329) (end 151.172799 104.155328) (width 0.3048) (layer F.Cu) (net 62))
 (segment (start 149.193399 105.445928) (end 150.2928 106.545329) (width 0.3048) (layer F.Cu) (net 61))
 (segment (start 149.193399 101.89473) (end 149.193399 105.445928) (width 0.3048) (layer F.Cu) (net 61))
 (segment (start 150.3228 100.765329) (end 149.193399 101.89473) (width 0.3048) (layer F.Cu) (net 61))
 (segment (start 148.632799 110.70533) (end 147.7528 111.585329) (width 0.3048) (layer F.Cu) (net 60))
 (segment (start 148.632799 104.155328) (end 148.632799 110.70533) (width 0.3048) (layer F.Cu) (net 60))
 (segment (start 147.7828 103.305329) (end 148.632799 104.155328) (width 0.3048) (layer F.Cu) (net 60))
 (segment (start 146.653399 105.445928) (end 147.7528 106.545329) (width 0.3048) (layer F.Cu) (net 59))
 (segment (start 146.653399 101.89473) (end 146.653399 105.445928) (width 0.3048) (layer F.Cu) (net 59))
 (segment (start 147.7828 100.765329) (end 146.653399 101.89473) (width 0.3048) (layer F.Cu) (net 59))
 (segment (start 146.092799 110.70533) (end 145.2128 111.585329) (width 0.3048) (layer F.Cu) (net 58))
 (segment (start 146.092799 104.155328) (end 146.092799 110.70533) (width 0.3048) (layer F.Cu) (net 58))
 (segment (start 145.2428 103.305329) (end 146.092799 104.155328) (width 0.3048) (layer F.Cu) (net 58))
 (segment (start 144.113399 105.445928) (end 145.2128 106.545329) (width 0.3048) (layer F.Cu) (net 57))
 (segment (start 144.113399 101.89473) (end 144.113399 105.445928) (width 0.3048) (layer F.Cu) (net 57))
 (segment (start 145.2428 100.765329) (end 144.113399 101.89473) (width 0.3048) (layer F.Cu) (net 57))
 (segment (start 143.552799 110.70533) (end 142.6728 111.585329) (width 0.3048) (layer F.Cu) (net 56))
 (segment (start 143.552799 104.155328) (end 143.552799 110.70533) (width 0.3048) (layer F.Cu) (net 56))
 (segment (start 142.7028 103.305329) (end 143.552799 104.155328) (width 0.3048) (layer F.Cu) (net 56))
 (segment (start 141.573399 105.445928) (end 142.6728 106.545329) (width 0.3048) (layer F.Cu) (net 55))
 (segment (start 142.7028 100.765329) (end 141.573399 101.89473) (width 0.3048) (layer F.Cu) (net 55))
 (segment (start 141.573399 101.89473) (end 141.573399 105.445928) (width 0.3048) (layer F.Cu) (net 55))
 (segment (start 141.012799 110.70533) (end 140.1328 111.585329) (width 0.3048) (layer F.Cu) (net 54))
 (segment (start 141.012799 104.155328) (end 141.012799 110.70533) (width 0.3048) (layer F.Cu) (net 54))
 (segment (start 140.1628 103.305329) (end 141.012799 104.155328) (width 0.3048) (layer F.Cu) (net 54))
 (segment (start 139.033399 105.445928) (end 140.1328 106.545329) (width 0.3048) (layer F.Cu) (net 53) (status 1000000))
 (segment (start 140.1628 100.765329) (end 139.033399 101.89473) (width 0.3048) (layer F.Cu) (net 53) (status 1000000))
 (segment (start 139.033399 101.89473) (end 139.033399 105.445928) (width 0.3048) (layer F.Cu) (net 53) (status 1000000))
 (segment (start 138.472799 110.70533) (end 137.5928 111.585329) (width 0.3048) (layer F.Cu) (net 52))
 (segment (start 138.472799 104.155328) (end 138.472799 110.70533) (width 0.3048) (layer F.Cu) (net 52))
 (segment (start 137.6228 103.305329) (end 138.472799 104.155328) (width 0.3048) (layer F.Cu) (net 52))
 (segment (start 136.493399 105.445928) (end 137.5928 106.545329) (width 0.3048) (layer F.Cu) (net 51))
 (segment (start 136.493399 101.89473) (end 136.493399 105.445928) (width 0.3048) (layer F.Cu) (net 51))
 (segment (start 137.6228 100.765329) (end 136.493399 101.89473) (width 0.3048) (layer F.Cu) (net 51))
 (segment (start 135.932799 110.70533) (end 135.0528 111.585329) (width 0.3048) (layer F.Cu) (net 50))
 (segment (start 135.932799 104.155328) (end 135.932799 110.70533) (width 0.3048) (layer F.Cu) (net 50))
 (segment (start 135.0828 103.305329) (end 135.932799 104.155328) (width 0.3048) (layer F.Cu) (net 50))
 (segment (start 133.953399 105.445928) (end 135.0528 106.545329) (width 0.3048) (layer F.Cu) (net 49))
 (segment (start 133.953399 101.89473) (end 133.953399 105.445928) (width 0.3048) (layer F.Cu) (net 49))
 (segment (start 135.0828 100.765329) (end 133.953399 101.89473) (width 0.3048) (layer F.Cu) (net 49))
 (segment (start 133.392799 110.70533) (end 132.5128 111.585329) (width 0.3048) (layer F.Cu) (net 48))
 (segment (start 133.392799 104.155328) (end 133.392799 110.70533) (width 0.3048) (layer F.Cu) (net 48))
 (segment (start 132.5428 103.305329) (end 133.392799 104.155328) (width 0.3048) (layer F.Cu) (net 48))
 (segment (start 131.413399 105.445928) (end 132.5128 106.545329) (width 0.3048) (layer F.Cu) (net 47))
 (segment (start 131.413399 101.89473) (end 131.413399 105.445928) (width 0.3048) (layer F.Cu) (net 47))
 (segment (start 132.5428 100.765329) (end 131.413399 101.89473) (width 0.3048) (layer F.Cu) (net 47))
 (segment (start 128.4928 104.815329) (end 122.2728 104.815329) (width 0.3048) (layer B.Cu) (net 46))
 (segment (start 130.0028 103.305329) (end 128.4928 104.815329) (width 0.3048) (layer B.Cu) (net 46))
 (segment (start 130.852799 110.70533) (end 129.9728 111.585329) (width 0.3048) (layer F.Cu) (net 46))
 (segment (start 130.852799 104.155328) (end 130.852799 110.70533) (width 0.3048) (layer F.Cu) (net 46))
 (segment (start 130.0028 103.305329) (end 130.852799 104.155328) (width 0.3048) (layer F.Cu) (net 46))
 (segment (start 122.2728 98.315329) (end 122.2728 98.524329) (width 0.3048) (layer B.Cu) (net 45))
 (segment (start 128.552799 99.315328) (end 130.0028 100.765329) (width 0.3048) (layer B.Cu) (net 45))
 (segment (start 123.272799 99.315328) (end 128.552799 99.315328) (width 0.3048) (layer B.Cu) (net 45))
 (segment (start 122.2728 98.315329) (end 123.272799 99.315328) (width 0.3048) (layer B.Cu) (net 45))
 (segment (start 128.873399 105.445928) (end 129.9728 106.545329) (width 0.3048) (layer F.Cu) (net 45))
 (segment (start 128.873399 101.89473) (end 128.873399 105.445928) (width 0.3048) (layer F.Cu) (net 45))
 (segment (start 130.0028 100.765329) (end 128.873399 101.89473) (width 0.3048) (layer F.Cu) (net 45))
 (segment (start 128.312799 110.70533) (end 127.4328 111.585329) (width 0.3048) (layer F.Cu) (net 44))
 (segment (start 128.312799 104.155328) (end 128.312799 110.70533) (width 0.3048) (layer F.Cu) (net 44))
 (segment (start 127.4628 103.305329) (end 128.312799 104.155328) (width 0.3048) (layer F.Cu) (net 44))
 (segment (start 126.333399 105.445928) (end 127.4328 106.545329) (width 0.3048) (layer F.Cu) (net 43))
 (segment (start 126.333399 101.89473) (end 126.333399 105.445928) (width 0.3048) (layer F.Cu) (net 43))
 (segment (start 127.4628 100.765329) (end 126.333399 101.89473) (width 0.3048) (layer F.Cu) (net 43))
 (segment (start 125.772799 110.70533) (end 124.8928 111.585329) (width 0.3048) (layer F.Cu) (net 42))
 (segment (start 125.772799 104.155328) (end 125.772799 110.70533) (width 0.3048) (layer F.Cu) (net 42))
 (segment (start 124.9228 103.305329) (end 125.772799 104.155328) (width 0.3048) (layer F.Cu) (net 42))
 (segment (start 123.793399 105.445928) (end 124.8928 106.545329) (width 0.3048) (layer F.Cu) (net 41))
 (segment (start 123.793399 101.89473) (end 123.793399 105.445928) (width 0.3048) (layer F.Cu) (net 41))
 (segment (start 124.9228 100.765329) (end 123.793399 101.89473) (width 0.3048) (layer F.Cu) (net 41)))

